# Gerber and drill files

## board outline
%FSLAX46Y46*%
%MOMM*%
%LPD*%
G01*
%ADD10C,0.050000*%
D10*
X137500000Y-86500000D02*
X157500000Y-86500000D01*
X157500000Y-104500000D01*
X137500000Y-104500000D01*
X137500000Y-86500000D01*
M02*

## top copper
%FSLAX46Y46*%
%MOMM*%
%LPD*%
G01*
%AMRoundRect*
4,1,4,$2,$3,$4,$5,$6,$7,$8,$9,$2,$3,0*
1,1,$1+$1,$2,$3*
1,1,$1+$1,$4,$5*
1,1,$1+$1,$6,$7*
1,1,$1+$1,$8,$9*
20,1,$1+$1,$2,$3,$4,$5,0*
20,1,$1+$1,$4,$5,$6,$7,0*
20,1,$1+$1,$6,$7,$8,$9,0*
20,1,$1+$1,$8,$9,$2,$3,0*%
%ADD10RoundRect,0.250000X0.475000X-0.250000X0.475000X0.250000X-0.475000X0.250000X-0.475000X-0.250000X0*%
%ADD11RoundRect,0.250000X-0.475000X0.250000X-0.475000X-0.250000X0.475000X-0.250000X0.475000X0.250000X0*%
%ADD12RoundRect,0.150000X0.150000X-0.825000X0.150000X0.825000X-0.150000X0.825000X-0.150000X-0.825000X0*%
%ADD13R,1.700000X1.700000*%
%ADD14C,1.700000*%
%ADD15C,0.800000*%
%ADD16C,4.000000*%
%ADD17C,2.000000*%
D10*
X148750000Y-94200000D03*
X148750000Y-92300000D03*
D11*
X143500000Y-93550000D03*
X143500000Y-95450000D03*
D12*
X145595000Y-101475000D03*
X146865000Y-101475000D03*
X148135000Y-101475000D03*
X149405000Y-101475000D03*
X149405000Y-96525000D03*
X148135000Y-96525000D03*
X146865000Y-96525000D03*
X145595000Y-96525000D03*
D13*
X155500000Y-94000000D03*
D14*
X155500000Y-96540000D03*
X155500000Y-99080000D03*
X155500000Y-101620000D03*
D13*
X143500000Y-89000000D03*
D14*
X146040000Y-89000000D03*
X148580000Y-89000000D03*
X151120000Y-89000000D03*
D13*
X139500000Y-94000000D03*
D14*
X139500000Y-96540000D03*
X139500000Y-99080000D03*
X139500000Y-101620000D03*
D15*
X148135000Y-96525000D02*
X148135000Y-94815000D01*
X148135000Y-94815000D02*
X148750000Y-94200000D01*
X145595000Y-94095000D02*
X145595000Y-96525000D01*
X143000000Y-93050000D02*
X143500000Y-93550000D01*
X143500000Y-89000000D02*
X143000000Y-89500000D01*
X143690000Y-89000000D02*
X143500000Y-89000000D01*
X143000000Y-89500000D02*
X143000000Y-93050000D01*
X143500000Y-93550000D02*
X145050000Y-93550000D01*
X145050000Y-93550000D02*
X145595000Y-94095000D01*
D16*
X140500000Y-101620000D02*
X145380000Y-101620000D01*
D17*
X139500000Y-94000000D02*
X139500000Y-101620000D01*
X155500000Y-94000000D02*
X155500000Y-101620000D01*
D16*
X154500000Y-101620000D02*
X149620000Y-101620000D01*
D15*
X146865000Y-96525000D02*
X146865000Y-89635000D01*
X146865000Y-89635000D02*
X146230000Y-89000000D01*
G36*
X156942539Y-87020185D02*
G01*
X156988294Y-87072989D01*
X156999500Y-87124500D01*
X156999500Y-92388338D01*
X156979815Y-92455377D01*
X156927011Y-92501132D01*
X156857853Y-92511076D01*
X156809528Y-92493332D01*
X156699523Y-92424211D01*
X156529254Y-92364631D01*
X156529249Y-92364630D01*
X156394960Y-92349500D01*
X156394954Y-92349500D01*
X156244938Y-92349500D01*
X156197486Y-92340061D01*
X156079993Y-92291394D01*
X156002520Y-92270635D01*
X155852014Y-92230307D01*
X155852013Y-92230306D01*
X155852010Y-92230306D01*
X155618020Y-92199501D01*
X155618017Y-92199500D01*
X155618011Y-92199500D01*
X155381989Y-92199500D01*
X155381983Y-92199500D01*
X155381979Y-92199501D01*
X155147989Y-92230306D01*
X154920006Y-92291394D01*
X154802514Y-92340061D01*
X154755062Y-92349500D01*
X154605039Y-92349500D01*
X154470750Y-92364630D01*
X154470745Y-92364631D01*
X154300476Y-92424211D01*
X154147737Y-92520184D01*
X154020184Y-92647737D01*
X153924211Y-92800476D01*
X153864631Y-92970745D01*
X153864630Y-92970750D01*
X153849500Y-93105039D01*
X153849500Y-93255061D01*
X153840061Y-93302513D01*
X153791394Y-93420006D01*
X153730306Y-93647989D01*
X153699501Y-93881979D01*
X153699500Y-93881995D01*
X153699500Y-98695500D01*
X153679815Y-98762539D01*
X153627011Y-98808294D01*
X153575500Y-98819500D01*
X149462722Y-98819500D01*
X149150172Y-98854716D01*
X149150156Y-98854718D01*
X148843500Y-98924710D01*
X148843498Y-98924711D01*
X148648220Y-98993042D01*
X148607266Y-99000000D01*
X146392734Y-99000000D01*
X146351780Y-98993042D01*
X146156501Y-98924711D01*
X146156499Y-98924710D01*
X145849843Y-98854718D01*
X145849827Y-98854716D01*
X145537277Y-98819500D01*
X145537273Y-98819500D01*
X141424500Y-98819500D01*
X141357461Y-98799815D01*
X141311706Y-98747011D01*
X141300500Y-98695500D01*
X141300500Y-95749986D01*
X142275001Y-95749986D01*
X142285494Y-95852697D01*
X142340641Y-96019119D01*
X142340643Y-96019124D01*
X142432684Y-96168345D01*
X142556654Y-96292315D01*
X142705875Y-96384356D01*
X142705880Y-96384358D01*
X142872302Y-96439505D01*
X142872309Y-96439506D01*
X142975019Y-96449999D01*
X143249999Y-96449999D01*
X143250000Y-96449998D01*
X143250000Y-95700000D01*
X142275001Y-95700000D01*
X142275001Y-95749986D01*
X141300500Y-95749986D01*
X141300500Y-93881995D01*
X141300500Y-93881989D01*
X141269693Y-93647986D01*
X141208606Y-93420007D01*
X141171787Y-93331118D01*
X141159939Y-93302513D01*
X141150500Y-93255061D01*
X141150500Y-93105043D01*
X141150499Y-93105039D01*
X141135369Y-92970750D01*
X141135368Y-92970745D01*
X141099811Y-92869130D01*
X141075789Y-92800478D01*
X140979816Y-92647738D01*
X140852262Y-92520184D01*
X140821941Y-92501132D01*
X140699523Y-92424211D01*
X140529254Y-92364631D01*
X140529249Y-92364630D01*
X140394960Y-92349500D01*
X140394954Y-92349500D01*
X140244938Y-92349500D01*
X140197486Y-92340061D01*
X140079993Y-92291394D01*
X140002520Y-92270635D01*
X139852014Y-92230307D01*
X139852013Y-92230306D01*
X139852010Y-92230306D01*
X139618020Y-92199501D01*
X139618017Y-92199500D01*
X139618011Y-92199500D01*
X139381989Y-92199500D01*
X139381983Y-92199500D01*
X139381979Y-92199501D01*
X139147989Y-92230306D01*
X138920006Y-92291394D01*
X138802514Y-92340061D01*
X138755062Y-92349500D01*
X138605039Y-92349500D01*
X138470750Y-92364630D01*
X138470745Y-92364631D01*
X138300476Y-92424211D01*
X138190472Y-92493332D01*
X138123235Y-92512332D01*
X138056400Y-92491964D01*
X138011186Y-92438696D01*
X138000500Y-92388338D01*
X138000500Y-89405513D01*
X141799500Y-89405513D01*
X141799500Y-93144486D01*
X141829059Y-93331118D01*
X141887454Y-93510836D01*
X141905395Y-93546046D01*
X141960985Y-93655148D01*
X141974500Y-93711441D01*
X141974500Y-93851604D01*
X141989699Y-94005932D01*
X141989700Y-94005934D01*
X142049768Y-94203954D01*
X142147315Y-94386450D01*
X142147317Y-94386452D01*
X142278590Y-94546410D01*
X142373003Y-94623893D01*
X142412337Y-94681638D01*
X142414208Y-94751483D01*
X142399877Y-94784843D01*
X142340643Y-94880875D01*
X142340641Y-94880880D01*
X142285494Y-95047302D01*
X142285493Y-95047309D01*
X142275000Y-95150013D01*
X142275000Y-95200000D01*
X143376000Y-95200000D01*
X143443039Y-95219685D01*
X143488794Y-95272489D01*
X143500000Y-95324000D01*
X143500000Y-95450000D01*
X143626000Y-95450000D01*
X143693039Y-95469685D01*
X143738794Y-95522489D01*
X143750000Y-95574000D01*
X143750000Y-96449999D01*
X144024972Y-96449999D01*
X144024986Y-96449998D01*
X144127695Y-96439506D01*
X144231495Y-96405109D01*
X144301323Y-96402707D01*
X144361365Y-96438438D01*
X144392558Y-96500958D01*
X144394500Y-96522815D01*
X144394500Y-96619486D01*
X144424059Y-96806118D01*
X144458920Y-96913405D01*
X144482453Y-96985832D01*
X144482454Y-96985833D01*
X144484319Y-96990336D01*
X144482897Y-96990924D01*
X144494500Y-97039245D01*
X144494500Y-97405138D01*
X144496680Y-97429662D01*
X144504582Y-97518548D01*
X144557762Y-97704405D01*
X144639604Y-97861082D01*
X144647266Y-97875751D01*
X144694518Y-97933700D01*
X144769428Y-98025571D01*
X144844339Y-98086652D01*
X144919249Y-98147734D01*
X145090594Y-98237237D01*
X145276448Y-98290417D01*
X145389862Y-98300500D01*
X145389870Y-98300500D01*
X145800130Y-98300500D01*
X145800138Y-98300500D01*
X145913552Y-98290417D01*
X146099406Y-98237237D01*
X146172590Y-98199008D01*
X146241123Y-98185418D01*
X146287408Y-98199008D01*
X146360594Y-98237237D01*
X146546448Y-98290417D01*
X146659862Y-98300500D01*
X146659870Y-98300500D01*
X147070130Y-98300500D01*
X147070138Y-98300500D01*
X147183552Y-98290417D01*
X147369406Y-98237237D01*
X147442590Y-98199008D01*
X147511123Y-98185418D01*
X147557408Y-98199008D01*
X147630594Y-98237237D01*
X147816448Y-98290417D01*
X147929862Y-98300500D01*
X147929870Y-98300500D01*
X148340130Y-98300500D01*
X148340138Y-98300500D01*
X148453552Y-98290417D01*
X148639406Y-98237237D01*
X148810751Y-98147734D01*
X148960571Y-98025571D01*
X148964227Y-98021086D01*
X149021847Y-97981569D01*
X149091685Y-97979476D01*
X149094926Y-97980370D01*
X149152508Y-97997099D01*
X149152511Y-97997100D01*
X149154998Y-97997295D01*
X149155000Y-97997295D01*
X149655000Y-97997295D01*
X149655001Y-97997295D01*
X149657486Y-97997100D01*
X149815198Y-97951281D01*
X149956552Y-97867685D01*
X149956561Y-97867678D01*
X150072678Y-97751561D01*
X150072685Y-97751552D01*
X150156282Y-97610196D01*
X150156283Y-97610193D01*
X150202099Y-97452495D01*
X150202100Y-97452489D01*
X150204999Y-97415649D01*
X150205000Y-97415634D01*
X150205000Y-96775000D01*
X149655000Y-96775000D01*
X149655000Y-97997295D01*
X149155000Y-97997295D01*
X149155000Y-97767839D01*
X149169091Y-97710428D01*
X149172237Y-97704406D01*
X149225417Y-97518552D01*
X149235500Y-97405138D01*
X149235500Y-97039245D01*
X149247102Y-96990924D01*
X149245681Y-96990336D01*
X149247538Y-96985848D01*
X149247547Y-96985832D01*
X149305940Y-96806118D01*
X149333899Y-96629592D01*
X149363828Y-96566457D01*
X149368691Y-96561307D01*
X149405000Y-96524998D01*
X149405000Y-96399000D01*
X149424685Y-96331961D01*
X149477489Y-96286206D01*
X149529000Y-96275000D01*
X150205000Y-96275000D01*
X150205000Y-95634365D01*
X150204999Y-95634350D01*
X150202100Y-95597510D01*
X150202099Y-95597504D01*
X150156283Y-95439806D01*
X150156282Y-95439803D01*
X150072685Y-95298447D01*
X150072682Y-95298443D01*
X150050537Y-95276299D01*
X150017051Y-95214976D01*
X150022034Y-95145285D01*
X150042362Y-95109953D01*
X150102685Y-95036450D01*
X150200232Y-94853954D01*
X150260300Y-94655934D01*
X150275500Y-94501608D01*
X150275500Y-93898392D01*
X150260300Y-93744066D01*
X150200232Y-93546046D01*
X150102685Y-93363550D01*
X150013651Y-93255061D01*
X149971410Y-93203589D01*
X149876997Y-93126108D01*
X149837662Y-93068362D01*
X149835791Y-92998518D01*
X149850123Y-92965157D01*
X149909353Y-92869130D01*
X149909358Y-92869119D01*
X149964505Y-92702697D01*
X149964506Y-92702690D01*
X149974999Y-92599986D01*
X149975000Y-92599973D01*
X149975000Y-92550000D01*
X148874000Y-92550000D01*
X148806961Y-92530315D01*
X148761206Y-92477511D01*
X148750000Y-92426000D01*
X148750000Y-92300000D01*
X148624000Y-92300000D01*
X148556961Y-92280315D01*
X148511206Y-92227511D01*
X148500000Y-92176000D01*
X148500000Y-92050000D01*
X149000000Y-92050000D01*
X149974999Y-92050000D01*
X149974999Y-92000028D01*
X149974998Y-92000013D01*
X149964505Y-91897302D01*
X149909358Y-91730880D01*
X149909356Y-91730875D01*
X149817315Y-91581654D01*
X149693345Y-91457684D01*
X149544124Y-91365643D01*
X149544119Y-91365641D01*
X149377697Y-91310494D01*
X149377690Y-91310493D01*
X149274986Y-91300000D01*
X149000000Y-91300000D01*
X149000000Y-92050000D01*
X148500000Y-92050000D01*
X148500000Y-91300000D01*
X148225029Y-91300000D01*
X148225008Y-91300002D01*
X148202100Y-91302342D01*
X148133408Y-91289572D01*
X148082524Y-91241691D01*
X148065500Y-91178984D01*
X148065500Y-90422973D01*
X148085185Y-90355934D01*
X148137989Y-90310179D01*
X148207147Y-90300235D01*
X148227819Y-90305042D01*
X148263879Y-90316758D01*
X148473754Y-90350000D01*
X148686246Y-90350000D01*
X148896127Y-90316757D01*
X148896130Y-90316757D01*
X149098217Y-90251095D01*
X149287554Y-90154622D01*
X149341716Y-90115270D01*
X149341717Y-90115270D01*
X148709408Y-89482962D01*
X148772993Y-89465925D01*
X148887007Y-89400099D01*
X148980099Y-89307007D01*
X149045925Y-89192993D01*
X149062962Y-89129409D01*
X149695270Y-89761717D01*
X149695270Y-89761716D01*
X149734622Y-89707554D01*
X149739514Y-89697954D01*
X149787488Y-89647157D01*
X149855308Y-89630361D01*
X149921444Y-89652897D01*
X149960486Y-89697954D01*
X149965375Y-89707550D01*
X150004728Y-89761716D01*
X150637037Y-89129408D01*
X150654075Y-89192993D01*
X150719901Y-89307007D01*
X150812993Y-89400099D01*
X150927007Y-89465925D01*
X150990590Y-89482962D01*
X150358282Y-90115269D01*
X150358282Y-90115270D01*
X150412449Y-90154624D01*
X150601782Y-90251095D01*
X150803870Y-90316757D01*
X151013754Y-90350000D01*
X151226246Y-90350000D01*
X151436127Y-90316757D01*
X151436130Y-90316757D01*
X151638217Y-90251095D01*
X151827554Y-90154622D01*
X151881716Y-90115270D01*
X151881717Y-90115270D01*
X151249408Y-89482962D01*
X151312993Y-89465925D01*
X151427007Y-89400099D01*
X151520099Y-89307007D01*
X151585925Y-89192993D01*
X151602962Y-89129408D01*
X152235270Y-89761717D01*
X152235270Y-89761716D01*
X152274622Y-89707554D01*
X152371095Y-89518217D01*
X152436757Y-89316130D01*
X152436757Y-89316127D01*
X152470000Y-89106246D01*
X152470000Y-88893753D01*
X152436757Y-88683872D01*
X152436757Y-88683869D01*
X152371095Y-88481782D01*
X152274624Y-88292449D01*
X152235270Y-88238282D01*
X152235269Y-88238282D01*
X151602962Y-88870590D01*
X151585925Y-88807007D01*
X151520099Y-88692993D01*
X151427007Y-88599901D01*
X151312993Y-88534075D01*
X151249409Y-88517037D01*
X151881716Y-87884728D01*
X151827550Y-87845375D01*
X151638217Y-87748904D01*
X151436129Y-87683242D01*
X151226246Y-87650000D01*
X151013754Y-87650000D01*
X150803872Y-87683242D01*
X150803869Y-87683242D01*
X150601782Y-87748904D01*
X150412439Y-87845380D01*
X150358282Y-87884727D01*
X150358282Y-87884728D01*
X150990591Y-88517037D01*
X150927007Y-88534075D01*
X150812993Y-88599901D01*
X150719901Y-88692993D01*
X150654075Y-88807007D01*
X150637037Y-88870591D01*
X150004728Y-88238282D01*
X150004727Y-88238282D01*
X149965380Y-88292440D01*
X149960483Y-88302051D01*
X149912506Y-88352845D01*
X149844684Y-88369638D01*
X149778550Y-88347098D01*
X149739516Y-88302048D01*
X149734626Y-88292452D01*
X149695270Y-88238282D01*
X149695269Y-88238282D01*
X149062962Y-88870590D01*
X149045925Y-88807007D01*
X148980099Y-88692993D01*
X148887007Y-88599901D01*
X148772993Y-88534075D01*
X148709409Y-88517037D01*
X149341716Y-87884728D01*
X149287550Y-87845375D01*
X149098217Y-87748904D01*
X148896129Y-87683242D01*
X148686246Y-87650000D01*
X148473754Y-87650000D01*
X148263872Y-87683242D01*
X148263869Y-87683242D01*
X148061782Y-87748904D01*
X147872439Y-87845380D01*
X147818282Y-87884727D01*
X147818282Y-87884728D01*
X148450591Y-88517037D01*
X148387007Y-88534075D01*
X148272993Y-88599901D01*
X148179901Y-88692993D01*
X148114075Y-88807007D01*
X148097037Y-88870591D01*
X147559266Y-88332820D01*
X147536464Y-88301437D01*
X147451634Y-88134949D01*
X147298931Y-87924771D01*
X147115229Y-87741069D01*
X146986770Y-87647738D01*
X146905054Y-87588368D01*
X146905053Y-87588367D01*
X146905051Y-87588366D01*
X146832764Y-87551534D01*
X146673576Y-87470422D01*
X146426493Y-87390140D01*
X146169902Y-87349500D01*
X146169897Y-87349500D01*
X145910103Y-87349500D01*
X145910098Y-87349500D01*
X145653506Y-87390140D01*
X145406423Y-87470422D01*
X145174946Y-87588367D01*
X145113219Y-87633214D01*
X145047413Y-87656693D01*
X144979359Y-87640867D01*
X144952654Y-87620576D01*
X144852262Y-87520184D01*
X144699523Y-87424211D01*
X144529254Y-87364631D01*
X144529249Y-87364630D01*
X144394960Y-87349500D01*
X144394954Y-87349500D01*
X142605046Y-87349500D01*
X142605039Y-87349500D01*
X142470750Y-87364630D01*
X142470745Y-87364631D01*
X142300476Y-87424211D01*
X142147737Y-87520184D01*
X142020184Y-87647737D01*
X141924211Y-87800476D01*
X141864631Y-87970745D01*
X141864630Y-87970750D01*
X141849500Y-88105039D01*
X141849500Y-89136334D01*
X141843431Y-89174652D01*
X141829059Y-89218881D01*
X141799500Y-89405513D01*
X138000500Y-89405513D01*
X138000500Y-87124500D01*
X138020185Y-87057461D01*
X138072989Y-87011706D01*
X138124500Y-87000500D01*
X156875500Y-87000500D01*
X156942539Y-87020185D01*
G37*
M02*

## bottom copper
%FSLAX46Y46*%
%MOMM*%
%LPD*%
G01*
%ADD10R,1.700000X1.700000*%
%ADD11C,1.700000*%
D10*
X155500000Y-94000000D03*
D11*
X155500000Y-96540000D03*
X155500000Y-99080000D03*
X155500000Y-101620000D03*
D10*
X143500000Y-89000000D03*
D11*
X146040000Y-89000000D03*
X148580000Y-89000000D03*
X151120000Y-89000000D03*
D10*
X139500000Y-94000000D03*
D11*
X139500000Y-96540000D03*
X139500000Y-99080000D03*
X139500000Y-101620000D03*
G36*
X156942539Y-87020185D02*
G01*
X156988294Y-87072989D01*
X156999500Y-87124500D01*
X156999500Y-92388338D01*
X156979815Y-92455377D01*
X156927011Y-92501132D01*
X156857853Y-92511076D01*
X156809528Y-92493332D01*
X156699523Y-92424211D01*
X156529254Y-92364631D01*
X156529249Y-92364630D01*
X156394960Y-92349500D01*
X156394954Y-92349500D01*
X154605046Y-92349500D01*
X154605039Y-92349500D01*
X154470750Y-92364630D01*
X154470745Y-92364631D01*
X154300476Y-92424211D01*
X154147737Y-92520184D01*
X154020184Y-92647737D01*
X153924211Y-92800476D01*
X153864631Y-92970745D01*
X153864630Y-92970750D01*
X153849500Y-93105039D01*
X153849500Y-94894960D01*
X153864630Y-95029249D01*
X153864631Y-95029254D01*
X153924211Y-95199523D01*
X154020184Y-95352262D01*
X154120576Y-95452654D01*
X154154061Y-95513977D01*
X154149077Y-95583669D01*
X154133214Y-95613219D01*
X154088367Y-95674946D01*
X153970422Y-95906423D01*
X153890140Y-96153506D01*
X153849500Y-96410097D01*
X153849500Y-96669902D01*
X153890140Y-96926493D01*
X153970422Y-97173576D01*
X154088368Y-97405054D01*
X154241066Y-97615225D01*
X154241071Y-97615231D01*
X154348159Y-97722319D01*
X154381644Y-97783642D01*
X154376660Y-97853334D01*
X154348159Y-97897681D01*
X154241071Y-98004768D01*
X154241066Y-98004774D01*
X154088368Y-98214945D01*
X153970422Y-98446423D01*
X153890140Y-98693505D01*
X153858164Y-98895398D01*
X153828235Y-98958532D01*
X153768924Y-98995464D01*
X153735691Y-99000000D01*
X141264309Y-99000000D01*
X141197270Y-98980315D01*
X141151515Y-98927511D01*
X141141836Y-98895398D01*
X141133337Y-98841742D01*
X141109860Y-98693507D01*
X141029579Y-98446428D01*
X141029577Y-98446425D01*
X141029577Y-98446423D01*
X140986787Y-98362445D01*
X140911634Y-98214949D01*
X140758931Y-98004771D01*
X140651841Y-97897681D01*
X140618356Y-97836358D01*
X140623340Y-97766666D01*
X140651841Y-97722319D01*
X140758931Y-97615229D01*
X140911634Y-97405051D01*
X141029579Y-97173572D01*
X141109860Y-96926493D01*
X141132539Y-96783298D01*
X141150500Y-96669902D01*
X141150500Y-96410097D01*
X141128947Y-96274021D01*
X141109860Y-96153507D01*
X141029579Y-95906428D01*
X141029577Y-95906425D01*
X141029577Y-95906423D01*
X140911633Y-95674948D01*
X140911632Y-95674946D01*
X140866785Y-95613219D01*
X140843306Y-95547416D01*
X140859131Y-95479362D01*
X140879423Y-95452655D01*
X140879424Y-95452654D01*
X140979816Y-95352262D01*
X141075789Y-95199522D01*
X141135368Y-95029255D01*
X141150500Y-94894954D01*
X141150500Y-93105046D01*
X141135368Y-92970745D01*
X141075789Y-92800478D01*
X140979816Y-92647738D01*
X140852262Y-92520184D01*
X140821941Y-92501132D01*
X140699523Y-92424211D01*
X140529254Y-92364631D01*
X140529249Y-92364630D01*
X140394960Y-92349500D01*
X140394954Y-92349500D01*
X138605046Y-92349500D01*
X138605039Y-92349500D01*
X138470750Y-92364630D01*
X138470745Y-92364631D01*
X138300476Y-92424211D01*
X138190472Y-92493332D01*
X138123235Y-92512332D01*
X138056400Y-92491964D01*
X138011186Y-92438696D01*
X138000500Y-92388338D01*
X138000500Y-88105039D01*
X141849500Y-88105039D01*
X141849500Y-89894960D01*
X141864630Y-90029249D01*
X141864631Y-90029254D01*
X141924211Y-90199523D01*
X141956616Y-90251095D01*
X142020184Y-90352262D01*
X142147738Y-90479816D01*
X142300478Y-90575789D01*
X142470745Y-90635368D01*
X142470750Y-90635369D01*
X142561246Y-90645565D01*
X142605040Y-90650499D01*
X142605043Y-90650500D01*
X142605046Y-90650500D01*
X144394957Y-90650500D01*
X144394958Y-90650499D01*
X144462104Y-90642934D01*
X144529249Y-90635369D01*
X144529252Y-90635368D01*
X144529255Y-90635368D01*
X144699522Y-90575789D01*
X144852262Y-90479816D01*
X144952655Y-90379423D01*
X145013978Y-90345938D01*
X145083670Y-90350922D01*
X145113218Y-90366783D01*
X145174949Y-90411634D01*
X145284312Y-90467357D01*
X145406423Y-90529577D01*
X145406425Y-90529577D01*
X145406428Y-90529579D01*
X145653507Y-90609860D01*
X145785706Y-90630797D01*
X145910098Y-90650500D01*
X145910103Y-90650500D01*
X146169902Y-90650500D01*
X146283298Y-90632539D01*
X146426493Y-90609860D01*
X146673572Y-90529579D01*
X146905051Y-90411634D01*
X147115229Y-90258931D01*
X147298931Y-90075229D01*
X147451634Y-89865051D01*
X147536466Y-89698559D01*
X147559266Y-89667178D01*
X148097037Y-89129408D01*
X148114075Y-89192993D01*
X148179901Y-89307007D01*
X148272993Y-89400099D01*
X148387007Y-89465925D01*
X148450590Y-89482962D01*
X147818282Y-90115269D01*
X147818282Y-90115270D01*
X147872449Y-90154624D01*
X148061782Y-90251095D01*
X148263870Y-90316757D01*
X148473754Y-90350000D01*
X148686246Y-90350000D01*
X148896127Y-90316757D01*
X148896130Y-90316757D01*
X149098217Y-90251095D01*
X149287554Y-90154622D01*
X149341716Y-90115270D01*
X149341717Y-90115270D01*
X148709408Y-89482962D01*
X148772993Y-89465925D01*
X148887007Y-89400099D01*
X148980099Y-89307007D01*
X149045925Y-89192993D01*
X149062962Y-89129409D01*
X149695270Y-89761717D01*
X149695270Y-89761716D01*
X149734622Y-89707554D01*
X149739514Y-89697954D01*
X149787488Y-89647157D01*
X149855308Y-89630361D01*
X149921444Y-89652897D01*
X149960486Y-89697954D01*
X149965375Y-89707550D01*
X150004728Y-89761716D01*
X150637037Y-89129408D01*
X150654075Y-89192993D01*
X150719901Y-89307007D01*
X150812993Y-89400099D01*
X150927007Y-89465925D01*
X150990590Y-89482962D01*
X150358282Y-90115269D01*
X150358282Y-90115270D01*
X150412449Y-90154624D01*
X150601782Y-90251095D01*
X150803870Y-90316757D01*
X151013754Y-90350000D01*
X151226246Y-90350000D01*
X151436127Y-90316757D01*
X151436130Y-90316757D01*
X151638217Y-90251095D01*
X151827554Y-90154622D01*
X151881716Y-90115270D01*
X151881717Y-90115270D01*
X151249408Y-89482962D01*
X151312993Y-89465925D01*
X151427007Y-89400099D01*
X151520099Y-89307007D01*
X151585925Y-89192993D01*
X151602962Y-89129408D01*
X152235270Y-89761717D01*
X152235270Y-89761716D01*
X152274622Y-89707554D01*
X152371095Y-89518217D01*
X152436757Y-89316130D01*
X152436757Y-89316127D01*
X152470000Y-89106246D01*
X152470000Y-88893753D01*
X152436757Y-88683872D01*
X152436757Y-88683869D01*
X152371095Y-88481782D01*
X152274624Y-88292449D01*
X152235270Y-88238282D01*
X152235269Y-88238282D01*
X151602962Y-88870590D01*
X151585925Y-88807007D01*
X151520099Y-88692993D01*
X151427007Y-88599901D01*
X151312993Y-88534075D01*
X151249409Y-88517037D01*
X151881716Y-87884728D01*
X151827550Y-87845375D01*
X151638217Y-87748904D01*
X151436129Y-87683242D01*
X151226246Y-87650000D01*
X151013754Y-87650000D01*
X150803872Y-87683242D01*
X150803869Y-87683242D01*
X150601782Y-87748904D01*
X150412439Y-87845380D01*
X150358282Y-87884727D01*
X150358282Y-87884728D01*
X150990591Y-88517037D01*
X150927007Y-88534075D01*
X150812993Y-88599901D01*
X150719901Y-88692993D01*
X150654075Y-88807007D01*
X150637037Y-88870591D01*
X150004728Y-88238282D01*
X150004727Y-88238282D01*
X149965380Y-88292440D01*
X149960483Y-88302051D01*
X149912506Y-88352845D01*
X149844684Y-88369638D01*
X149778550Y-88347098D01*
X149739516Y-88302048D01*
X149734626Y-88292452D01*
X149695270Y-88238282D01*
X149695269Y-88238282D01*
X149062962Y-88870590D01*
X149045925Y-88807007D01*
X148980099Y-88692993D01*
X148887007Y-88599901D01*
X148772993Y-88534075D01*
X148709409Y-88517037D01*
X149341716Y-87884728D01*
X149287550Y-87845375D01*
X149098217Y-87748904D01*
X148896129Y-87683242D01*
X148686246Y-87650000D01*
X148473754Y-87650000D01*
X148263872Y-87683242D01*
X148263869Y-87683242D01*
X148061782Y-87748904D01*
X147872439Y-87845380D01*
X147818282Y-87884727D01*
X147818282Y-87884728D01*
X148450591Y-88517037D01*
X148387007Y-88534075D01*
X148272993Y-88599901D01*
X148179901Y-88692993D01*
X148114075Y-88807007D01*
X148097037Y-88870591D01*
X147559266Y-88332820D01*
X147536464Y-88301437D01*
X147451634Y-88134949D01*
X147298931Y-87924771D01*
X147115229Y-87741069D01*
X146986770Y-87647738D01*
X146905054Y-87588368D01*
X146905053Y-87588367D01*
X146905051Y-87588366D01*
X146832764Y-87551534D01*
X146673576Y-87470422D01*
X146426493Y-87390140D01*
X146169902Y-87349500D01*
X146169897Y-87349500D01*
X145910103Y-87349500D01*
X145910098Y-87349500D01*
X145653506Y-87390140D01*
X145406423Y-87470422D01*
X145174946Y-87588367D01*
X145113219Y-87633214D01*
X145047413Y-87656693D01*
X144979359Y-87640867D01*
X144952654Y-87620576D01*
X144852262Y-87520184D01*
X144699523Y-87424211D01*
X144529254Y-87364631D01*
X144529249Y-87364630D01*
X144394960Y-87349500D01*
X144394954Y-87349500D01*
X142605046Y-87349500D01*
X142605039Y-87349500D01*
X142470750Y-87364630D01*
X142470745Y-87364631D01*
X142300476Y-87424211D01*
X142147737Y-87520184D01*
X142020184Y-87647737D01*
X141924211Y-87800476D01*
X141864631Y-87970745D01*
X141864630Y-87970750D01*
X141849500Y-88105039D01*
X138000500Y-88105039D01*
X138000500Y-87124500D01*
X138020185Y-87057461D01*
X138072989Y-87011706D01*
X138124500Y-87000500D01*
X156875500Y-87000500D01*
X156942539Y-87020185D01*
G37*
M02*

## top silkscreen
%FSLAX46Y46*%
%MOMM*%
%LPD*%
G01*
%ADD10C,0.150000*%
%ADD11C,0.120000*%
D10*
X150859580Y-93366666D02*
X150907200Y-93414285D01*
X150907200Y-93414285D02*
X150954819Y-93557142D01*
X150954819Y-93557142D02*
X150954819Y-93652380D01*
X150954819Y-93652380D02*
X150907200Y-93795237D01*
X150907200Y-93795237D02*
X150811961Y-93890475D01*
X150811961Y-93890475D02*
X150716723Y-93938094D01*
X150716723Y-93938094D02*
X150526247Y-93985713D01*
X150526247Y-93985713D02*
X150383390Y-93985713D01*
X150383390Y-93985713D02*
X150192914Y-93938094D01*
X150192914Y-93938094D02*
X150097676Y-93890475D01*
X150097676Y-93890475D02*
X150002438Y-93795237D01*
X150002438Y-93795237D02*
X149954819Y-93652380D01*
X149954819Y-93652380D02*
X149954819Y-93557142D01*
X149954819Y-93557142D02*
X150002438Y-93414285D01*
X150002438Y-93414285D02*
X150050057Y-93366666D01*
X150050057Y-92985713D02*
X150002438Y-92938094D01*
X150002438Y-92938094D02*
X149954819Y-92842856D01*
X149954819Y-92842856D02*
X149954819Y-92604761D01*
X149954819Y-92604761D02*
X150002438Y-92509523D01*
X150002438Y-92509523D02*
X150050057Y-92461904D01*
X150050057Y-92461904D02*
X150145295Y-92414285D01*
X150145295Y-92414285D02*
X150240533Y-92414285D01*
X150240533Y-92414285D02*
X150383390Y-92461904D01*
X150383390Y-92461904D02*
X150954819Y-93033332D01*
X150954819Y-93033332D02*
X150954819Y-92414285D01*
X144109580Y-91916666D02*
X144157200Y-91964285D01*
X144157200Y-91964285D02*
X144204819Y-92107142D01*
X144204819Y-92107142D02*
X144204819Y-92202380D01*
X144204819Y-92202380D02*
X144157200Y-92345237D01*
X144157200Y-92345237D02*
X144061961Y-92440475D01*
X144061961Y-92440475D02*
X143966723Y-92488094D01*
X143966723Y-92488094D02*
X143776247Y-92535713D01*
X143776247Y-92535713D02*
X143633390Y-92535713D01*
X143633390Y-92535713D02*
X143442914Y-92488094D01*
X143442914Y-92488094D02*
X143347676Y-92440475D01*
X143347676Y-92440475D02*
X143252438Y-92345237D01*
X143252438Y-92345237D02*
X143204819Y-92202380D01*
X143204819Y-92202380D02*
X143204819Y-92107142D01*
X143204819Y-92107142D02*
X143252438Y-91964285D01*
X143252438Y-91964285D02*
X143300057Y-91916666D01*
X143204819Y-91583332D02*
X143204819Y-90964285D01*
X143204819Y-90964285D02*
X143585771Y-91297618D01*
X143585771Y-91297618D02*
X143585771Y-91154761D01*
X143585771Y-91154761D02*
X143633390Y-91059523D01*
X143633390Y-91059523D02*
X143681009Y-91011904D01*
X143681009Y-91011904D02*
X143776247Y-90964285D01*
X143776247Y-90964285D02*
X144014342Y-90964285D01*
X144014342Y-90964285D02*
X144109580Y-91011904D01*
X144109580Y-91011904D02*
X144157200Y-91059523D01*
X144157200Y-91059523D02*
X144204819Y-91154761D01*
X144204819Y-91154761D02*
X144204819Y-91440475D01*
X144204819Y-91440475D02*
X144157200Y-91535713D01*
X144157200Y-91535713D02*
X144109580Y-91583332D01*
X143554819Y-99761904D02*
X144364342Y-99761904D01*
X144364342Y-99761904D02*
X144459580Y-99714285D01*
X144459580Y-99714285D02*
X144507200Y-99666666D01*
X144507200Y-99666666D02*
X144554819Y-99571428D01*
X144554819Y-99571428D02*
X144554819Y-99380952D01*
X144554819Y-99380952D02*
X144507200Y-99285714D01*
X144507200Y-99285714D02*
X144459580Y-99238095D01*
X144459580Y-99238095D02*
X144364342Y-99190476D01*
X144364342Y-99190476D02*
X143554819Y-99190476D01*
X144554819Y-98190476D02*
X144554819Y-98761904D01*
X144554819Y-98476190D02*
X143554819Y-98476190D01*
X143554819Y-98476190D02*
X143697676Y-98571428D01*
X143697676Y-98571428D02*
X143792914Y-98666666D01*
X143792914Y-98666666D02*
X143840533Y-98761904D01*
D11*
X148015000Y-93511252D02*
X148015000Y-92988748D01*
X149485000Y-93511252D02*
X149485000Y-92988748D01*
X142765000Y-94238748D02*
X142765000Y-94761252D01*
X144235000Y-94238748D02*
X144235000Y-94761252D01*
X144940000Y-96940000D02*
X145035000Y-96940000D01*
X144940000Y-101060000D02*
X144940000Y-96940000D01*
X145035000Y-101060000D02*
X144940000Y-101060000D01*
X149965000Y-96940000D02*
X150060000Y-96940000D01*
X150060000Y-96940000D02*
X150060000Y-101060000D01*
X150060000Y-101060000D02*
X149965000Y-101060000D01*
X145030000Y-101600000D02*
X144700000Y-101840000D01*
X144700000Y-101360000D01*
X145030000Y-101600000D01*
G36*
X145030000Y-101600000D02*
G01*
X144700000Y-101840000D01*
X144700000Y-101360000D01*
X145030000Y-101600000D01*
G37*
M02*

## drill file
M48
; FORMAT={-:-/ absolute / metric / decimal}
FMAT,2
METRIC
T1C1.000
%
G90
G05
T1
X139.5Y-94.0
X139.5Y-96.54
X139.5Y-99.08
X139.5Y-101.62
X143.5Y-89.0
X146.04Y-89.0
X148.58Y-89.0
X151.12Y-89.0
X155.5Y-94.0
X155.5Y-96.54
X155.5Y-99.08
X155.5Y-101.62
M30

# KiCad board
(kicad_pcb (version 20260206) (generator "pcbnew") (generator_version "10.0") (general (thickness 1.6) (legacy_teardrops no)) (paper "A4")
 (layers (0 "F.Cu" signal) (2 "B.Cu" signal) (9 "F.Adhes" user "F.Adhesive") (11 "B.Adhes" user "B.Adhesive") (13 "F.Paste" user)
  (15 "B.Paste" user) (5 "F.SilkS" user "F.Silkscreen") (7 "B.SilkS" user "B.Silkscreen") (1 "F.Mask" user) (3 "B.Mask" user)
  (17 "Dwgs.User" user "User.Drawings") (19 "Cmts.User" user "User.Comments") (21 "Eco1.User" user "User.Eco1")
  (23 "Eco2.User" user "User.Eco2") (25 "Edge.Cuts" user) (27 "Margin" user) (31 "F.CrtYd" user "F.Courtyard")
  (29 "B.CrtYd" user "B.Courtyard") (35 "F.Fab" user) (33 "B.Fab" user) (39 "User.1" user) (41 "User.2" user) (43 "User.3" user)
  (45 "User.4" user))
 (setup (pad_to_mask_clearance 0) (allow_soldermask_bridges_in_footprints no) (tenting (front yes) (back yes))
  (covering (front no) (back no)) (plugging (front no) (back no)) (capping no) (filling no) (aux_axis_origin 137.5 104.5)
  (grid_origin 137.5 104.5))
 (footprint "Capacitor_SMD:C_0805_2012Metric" (layer "F.Cu") (at 148.75 93.25 90)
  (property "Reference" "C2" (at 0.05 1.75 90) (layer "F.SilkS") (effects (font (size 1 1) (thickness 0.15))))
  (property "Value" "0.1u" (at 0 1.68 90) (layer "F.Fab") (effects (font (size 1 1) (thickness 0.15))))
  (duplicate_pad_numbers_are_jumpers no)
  (fp_line (start -0.261252 -0.735) (end 0.261252 -0.735) (stroke (width 0.12) (type solid)) (layer "F.SilkS"))
  (fp_line (start -0.261252 0.735) (end 0.261252 0.735) (stroke (width 0.12) (type solid)) (layer "F.SilkS"))
  (pad "1" smd roundrect (at -0.95 0 90) (size 1 1.45) (layers "F.Cu" "F.Mask" "F.Paste") (roundrect_rratio 0.25) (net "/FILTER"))
  (pad "2" smd roundrect (at 0.95 0 90) (size 1 1.45) (layers "F.Cu" "F.Mask" "F.Paste") (roundrect_rratio 0.25) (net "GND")))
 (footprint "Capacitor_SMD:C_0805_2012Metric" (layer "F.Cu") (at 143.5 94.5 -90)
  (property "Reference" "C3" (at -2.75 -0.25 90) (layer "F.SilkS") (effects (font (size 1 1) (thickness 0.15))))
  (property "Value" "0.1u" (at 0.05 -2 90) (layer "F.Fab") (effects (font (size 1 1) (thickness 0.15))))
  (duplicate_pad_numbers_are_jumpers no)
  (fp_line (start -0.261252 0.735) (end 0.261252 0.735) (stroke (width 0.12) (type solid)) (layer "F.SilkS"))
  (fp_line (start -0.261252 -0.735) (end 0.261252 -0.735) (stroke (width 0.12) (type solid)) (layer "F.SilkS"))
  (pad "1" smd roundrect (at -0.95 0 270) (size 1 1.45) (layers "F.Cu" "F.Mask" "F.Paste") (roundrect_rratio 0.25) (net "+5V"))
  (pad "2" smd roundrect (at 0.95 0 270) (size 1 1.45) (layers "F.Cu" "F.Mask" "F.Paste") (roundrect_rratio 0.25) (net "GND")))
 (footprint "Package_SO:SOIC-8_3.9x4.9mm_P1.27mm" (layer "F.Cu") (at 147.5 99 90)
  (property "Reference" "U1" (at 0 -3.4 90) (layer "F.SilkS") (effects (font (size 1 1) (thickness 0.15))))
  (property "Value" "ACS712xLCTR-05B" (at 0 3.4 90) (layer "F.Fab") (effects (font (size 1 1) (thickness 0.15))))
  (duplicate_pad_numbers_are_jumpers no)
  (fp_line (start 2.06 -2.56) (end 2.06 -2.465) (stroke (width 0.12) (type solid)) (layer "F.SilkS"))
  (fp_line (start -2.06 -2.56) (end 2.06 -2.56) (stroke (width 0.12) (type solid)) (layer "F.SilkS"))
  (fp_line (start -2.06 -2.465) (end -2.06 -2.56) (stroke (width 0.12) (type solid)) (layer "F.SilkS"))
  (fp_line (start 2.06 2.465) (end 2.06 2.56) (stroke (width 0.12) (type solid)) (layer "F.SilkS"))
  (fp_line (start 2.06 2.56) (end -2.06 2.56) (stroke (width 0.12) (type solid)) (layer "F.SilkS"))
  (fp_line (start -2.06 2.56) (end -2.06 2.465) (stroke (width 0.12) (type solid)) (layer "F.SilkS"))
  (fp_poly (pts (xy -2.6 -2.47) (xy -2.84 -2.8) (xy -2.36 -2.8)) (stroke (width 0.12) (type solid)) (fill yes) (layer "F.SilkS"))
  (pad "1" smd roundrect (at -2.475 -1.905 90) (size 1.95 0.6) (layers "F.Cu" "F.Mask" "F.Paste") (roundrect_rratio 0.25) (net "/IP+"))
  (pad "2" smd roundrect (at -2.475 -0.635 90) (size 1.95 0.6) (layers "F.Cu" "F.Mask" "F.Paste") (roundrect_rratio 0.25) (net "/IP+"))
  (pad "3" smd roundrect (at -2.475 0.635 90) (size 1.95 0.6) (layers "F.Cu" "F.Mask" "F.Paste") (roundrect_rratio 0.25) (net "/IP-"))
  (pad "4" smd roundrect (at -2.475 1.905 90) (size 1.95 0.6) (layers "F.Cu" "F.Mask" "F.Paste") (roundrect_rratio 0.25) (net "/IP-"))
  (pad "5" smd roundrect (at 2.475 1.905 90) (size 1.95 0.6) (layers "F.Cu" "F.Mask" "F.Paste") (roundrect_rratio 0.25) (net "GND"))
  (pad "6" smd roundrect (at 2.475 0.635 90) (size 1.95 0.6) (layers "F.Cu" "F.Mask" "F.Paste") (roundrect_rratio 0.25) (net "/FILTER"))
  (pad "7" smd roundrect (at 2.475 -0.635 90) (size 1.95 0.6) (layers "F.Cu" "F.Mask" "F.Paste") (roundrect_rratio 0.25) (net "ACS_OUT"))
  (pad "8" smd roundrect (at 2.475 -1.905 90) (size 1.95 0.6) (layers "F.Cu" "F.Mask" "F.Paste") (roundrect_rratio 0.25) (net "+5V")))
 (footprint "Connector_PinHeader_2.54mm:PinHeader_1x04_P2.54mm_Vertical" (layer "B.Cu") (at 155.5 94 180)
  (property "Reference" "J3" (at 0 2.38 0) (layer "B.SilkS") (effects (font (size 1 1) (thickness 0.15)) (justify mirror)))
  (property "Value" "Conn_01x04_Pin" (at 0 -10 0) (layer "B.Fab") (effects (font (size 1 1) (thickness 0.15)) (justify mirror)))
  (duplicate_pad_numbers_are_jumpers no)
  (pad "1" thru_hole rect (at 0 0 180) (size 1.7 1.7) (drill 1) (layers "*.Cu" "*.Mask") (remove_unused_layers no) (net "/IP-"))
  (pad "2" thru_hole circle (at 0 -2.54 180) (size 1.7 1.7) (drill 1) (layers "*.Cu" "*.Mask") (remove_unused_layers no) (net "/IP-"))
  (pad "3" thru_hole circle (at 0 -5.08 180) (size 1.7 1.7) (drill 1) (layers "*.Cu" "*.Mask") (remove_unused_layers no) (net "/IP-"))
  (pad "4" thru_hole circle (at 0 -7.62 180) (size 1.7 1.7) (drill 1) (layers "*.Cu" "*.Mask") (remove_unused_layers no) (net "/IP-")))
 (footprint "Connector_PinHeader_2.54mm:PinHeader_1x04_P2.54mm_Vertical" (layer "B.Cu") (at 143.5 89 -90)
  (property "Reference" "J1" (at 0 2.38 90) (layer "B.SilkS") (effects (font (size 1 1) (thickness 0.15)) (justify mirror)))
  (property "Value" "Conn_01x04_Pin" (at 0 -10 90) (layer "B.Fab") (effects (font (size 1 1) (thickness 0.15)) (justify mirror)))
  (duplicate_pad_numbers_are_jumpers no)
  (pad "1" thru_hole rect (at 0 0 270) (size 1.7 1.7) (drill 1) (layers "*.Cu" "*.Mask") (remove_unused_layers no) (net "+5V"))
  (pad "2" thru_hole circle (at 0 -2.54 270) (size 1.7 1.7) (drill 1) (layers "*.Cu" "*.Mask") (remove_unused_layers no) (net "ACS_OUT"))
  (pad "3" thru_hole circle (at 0 -5.08 270) (size 1.7 1.7) (drill 1) (layers "*.Cu" "*.Mask") (remove_unused_layers no) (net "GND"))
  (pad "4" thru_hole circle (at 0 -7.62 270) (size 1.7 1.7) (drill 1) (layers "*.Cu" "*.Mask") (remove_unused_layers no) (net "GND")))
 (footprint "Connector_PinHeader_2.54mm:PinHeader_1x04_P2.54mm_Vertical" (layer "B.Cu") (at 139.5 94 180)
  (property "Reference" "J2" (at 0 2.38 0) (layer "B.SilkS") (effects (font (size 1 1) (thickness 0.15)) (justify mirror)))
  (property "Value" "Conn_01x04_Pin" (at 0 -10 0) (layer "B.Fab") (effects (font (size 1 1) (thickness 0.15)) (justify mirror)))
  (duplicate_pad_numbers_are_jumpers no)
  (pad "1" thru_hole rect (at 0 0 180) (size 1.7 1.7) (drill 1) (layers "*.Cu" "*.Mask") (remove_unused_layers no) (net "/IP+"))
  (pad "2" thru_hole circle (at 0 -2.54 180) (size 1.7 1.7) (drill 1) (layers "*.Cu" "*.Mask") (remove_unused_layers no) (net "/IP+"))
  (pad "3" thru_hole circle (at 0 -5.08 180) (size 1.7 1.7) (drill 1) (layers "*.Cu" "*.Mask") (remove_unused_layers no) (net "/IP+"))
  (pad "4" thru_hole circle (at 0 -7.62 180) (size 1.7 1.7) (drill 1) (layers "*.Cu" "*.Mask") (remove_unused_layers no) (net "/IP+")))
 (gr_rect (start 137.5 86.5) (end 157.5 104.5) (stroke (width 0.05) (type solid)) (fill no) (layer "Edge.Cuts"))
 (segment (start 148.135 96.525) (end 148.135 94.815) (width 0.8) (layer "F.Cu") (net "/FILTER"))
 (segment (start 148.135 94.815) (end 148.75 94.2) (width 0.8) (layer "F.Cu") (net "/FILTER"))
 (segment (start 145.595 94.095) (end 145.595 96.525) (width 0.8) (layer "F.Cu") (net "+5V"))
 (segment (start 143 93.05) (end 143.5 93.55) (width 0.8) (layer "F.Cu") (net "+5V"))
 (segment (start 143.5 89) (end 143 89.5) (width 0.8) (layer "F.Cu") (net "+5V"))
 (segment (start 143.69 89) (end 143.5 89) (width 0.8) (layer "F.Cu") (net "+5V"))
 (segment (start 143 89.5) (end 143 93.05) (width 0.8) (layer "F.Cu") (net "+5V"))
 (segment (start 143.5 93.55) (end 145.05 93.55) (width 0.8) (layer "F.Cu") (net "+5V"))
 (segment (start 145.05 93.55) (end 145.595 94.095) (width 0.8) (layer "F.Cu") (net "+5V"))
 (segment (start 140.5 101.62) (end 145.38 101.62) (width 4) (layer "F.Cu") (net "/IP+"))
 (segment (start 139.5 94) (end 139.5 101.62) (width 2) (layer "F.Cu") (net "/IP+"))
 (segment (start 155.5 94) (end 155.5 101.62) (width 2) (layer "F.Cu") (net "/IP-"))
 (segment (start 154.5 101.62) (end 149.62 101.62) (width 4) (layer "F.Cu") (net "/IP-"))
 (segment (start 146.865 96.525) (end 146.865 89.635) (width 0.8) (layer "F.Cu") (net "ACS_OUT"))
 (segment (start 146.865 89.635) (end 146.23 89) (width 0.8) (layer "F.Cu") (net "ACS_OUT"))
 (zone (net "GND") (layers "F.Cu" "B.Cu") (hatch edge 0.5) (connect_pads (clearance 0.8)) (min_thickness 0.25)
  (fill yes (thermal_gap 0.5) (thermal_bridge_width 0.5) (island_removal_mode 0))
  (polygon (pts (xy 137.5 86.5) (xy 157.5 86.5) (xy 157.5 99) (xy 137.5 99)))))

